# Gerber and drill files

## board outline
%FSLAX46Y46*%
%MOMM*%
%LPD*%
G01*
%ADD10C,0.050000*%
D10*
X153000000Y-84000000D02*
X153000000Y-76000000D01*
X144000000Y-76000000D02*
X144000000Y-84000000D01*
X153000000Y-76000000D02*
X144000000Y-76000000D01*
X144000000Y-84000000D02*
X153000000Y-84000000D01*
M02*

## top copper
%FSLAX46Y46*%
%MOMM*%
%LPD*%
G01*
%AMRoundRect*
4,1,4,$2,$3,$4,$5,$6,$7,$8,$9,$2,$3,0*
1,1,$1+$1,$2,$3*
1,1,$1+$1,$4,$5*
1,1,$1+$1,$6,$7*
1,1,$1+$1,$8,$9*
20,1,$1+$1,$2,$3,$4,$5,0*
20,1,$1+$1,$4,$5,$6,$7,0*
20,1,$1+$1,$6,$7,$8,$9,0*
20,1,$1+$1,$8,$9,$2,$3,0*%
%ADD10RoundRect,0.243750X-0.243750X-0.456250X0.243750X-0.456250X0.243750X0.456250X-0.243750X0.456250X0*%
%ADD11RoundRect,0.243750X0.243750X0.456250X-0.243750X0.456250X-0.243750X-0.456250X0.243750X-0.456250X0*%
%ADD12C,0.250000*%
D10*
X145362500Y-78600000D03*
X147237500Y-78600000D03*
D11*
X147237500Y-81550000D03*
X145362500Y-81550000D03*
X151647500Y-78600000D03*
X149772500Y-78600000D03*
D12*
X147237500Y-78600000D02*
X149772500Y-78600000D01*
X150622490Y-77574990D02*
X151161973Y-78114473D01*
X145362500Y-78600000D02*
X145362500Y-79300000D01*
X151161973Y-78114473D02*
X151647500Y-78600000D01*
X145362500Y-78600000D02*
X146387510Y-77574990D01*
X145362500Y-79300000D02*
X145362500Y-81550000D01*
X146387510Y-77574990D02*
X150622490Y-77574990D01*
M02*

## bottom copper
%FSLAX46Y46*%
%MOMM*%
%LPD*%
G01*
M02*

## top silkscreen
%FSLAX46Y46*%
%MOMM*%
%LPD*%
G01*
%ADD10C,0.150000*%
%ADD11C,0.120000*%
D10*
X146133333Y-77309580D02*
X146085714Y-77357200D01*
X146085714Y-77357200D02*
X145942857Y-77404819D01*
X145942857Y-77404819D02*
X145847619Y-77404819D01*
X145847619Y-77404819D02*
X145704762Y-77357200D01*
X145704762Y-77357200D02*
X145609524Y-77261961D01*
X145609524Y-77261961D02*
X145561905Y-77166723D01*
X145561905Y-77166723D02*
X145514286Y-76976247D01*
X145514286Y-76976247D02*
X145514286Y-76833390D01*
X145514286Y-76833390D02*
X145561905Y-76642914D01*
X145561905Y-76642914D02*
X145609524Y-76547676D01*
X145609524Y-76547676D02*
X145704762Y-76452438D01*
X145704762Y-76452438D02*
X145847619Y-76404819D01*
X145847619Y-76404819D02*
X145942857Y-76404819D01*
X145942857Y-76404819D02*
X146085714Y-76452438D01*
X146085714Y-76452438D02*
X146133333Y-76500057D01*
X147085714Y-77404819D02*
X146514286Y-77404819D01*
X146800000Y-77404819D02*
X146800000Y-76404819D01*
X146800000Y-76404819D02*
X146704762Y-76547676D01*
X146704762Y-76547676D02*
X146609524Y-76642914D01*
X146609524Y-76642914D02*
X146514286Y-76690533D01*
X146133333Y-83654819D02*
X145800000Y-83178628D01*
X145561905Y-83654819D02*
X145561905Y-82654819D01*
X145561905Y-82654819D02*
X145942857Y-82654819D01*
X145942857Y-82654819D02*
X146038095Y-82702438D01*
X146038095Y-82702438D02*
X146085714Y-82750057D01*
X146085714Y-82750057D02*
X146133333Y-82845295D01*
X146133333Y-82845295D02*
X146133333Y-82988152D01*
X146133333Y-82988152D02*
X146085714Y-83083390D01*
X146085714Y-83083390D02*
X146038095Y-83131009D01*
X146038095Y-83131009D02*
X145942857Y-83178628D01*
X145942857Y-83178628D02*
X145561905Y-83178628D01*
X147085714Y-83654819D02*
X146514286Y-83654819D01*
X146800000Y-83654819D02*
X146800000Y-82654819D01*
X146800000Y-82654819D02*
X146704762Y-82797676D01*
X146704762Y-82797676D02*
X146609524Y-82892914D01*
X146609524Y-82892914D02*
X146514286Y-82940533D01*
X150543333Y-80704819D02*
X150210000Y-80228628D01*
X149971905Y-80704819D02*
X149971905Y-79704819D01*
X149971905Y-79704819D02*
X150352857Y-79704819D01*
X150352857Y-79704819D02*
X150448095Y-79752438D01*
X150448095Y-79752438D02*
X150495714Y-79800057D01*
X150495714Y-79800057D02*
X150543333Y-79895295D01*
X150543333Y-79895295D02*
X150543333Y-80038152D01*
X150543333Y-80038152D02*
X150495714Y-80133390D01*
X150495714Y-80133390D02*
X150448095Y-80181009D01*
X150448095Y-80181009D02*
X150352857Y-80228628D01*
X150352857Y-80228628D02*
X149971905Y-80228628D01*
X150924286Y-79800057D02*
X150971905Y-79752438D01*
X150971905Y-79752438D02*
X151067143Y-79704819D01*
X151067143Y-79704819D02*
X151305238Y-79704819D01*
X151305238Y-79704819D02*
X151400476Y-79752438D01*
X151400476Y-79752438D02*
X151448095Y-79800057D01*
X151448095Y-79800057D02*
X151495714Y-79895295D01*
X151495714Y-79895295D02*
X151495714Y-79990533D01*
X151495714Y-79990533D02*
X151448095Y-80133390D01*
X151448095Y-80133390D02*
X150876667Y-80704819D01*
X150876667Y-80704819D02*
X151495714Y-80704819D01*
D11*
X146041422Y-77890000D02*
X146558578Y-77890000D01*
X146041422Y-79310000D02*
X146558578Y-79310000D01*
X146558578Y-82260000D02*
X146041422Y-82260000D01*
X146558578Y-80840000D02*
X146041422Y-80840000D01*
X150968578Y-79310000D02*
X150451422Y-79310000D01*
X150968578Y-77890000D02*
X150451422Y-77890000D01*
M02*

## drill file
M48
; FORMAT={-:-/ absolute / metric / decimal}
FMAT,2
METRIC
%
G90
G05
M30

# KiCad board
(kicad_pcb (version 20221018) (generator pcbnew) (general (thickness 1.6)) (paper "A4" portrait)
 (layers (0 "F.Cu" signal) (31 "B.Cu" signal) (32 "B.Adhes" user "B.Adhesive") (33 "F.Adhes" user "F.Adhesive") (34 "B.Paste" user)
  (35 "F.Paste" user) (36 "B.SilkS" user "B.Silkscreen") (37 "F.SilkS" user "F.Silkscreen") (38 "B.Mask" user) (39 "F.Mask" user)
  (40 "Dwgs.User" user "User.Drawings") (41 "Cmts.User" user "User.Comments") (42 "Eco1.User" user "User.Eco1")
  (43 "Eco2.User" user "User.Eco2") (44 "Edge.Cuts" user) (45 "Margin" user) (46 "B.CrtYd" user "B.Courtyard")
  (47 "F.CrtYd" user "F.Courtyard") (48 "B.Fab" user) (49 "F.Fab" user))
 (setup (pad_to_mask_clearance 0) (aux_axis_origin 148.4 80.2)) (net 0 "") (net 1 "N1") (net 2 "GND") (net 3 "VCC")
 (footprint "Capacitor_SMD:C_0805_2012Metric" (layer "F.Cu") (at 146.3 78.6)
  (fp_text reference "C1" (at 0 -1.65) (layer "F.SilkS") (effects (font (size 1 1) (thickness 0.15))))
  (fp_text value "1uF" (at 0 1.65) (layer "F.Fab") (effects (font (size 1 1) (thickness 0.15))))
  (fp_line (start -0.258578 -0.71) (end 0.258578 -0.71) (stroke (width 0.12) (type solid)) (layer "F.SilkS"))
  (fp_line (start -0.258578 0.71) (end 0.258578 0.71) (stroke (width 0.12) (type solid)) (layer "F.SilkS"))
  (pad "1" smd roundrect (at -0.9375 0) (size 0.975 1.4) (layers "F.Cu" "F.Paste" "F.Mask") (roundrect_rratio 0.25) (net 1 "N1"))
  (pad "2" smd roundrect (at 0.9375 0) (size 0.975 1.4) (layers "F.Cu" "F.Paste" "F.Mask") (roundrect_rratio 0.25) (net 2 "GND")))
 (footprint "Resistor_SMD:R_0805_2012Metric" (layer "F.Cu") (at 146.3 81.55 180)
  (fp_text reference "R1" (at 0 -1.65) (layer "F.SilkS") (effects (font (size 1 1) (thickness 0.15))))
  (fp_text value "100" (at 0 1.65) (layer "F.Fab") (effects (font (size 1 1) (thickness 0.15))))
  (fp_line (start -0.258578 -0.71) (end 0.258578 -0.71) (stroke (width 0.12) (type solid)) (layer "F.SilkS"))
  (fp_line (start -0.258578 0.71) (end 0.258578 0.71) (stroke (width 0.12) (type solid)) (layer "F.SilkS"))
  (pad "1" smd roundrect (at -0.9375 0 180) (size 0.975 1.4) (layers "F.Cu" "F.Paste" "F.Mask") (roundrect_rratio 0.25) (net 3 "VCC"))
  (pad "2" smd roundrect (at 0.9375 0 180) (size 0.975 1.4) (layers "F.Cu" "F.Paste" "F.Mask") (roundrect_rratio 0.25) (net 1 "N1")))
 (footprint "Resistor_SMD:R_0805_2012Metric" (layer "F.Cu") (at 150.71 78.6 180)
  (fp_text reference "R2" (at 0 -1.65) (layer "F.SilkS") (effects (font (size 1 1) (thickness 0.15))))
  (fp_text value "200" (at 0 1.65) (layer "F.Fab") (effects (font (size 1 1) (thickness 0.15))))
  (fp_line (start -0.258578 -0.71) (end 0.258578 -0.71) (stroke (width 0.12) (type solid)) (layer "F.SilkS"))
  (fp_line (start -0.258578 0.71) (end 0.258578 0.71) (stroke (width 0.12) (type solid)) (layer "F.SilkS"))
  (pad "1" smd roundrect (at -0.9375 0 180) (size 0.975 1.4) (layers "F.Cu" "F.Paste" "F.Mask") (roundrect_rratio 0.25) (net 1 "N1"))
  (pad "2" smd roundrect (at 0.9375 0 180) (size 0.975 1.4) (layers "F.Cu" "F.Paste" "F.Mask") (roundrect_rratio 0.25) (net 2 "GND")))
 (gr_line (start 153 84) (end 153 76) (stroke (width 0.05) (type solid)) (layer "Edge.Cuts"))
 (gr_line (start 144 76) (end 144 84) (stroke (width 0.05) (type solid)) (layer "Edge.Cuts"))
 (gr_line (start 153 76) (end 144 76) (stroke (width 0.05) (type solid)) (layer "Edge.Cuts"))
 (gr_line (start 144 84) (end 153 84) (stroke (width 0.05) (type solid)) (layer "Edge.Cuts"))
 (segment (start 147.2375 78.6) (end 149.7725 78.6) (width 0.25) (layer "F.Cu") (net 2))
 (segment (start 150.62249 77.57499) (end 151.161973 78.114473) (width 0.25) (layer "F.Cu") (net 1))
 (segment (start 145.3625 78.6) (end 145.3625 79.3) (width 0.25) (layer "F.Cu") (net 1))
 (segment (start 151.161973 78.114473) (end 151.6475 78.6) (width 0.25) (layer "F.Cu") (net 1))
 (segment (start 145.3625 78.6) (end 146.38751 77.57499) (width 0.25) (layer "F.Cu") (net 1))
 (segment (start 145.3625 79.3) (end 145.3625 81.55) (width 0.25) (layer "F.Cu") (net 1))
 (segment (start 146.38751 77.57499) (end 150.62249 77.57499) (width 0.25) (layer "F.Cu") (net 1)))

